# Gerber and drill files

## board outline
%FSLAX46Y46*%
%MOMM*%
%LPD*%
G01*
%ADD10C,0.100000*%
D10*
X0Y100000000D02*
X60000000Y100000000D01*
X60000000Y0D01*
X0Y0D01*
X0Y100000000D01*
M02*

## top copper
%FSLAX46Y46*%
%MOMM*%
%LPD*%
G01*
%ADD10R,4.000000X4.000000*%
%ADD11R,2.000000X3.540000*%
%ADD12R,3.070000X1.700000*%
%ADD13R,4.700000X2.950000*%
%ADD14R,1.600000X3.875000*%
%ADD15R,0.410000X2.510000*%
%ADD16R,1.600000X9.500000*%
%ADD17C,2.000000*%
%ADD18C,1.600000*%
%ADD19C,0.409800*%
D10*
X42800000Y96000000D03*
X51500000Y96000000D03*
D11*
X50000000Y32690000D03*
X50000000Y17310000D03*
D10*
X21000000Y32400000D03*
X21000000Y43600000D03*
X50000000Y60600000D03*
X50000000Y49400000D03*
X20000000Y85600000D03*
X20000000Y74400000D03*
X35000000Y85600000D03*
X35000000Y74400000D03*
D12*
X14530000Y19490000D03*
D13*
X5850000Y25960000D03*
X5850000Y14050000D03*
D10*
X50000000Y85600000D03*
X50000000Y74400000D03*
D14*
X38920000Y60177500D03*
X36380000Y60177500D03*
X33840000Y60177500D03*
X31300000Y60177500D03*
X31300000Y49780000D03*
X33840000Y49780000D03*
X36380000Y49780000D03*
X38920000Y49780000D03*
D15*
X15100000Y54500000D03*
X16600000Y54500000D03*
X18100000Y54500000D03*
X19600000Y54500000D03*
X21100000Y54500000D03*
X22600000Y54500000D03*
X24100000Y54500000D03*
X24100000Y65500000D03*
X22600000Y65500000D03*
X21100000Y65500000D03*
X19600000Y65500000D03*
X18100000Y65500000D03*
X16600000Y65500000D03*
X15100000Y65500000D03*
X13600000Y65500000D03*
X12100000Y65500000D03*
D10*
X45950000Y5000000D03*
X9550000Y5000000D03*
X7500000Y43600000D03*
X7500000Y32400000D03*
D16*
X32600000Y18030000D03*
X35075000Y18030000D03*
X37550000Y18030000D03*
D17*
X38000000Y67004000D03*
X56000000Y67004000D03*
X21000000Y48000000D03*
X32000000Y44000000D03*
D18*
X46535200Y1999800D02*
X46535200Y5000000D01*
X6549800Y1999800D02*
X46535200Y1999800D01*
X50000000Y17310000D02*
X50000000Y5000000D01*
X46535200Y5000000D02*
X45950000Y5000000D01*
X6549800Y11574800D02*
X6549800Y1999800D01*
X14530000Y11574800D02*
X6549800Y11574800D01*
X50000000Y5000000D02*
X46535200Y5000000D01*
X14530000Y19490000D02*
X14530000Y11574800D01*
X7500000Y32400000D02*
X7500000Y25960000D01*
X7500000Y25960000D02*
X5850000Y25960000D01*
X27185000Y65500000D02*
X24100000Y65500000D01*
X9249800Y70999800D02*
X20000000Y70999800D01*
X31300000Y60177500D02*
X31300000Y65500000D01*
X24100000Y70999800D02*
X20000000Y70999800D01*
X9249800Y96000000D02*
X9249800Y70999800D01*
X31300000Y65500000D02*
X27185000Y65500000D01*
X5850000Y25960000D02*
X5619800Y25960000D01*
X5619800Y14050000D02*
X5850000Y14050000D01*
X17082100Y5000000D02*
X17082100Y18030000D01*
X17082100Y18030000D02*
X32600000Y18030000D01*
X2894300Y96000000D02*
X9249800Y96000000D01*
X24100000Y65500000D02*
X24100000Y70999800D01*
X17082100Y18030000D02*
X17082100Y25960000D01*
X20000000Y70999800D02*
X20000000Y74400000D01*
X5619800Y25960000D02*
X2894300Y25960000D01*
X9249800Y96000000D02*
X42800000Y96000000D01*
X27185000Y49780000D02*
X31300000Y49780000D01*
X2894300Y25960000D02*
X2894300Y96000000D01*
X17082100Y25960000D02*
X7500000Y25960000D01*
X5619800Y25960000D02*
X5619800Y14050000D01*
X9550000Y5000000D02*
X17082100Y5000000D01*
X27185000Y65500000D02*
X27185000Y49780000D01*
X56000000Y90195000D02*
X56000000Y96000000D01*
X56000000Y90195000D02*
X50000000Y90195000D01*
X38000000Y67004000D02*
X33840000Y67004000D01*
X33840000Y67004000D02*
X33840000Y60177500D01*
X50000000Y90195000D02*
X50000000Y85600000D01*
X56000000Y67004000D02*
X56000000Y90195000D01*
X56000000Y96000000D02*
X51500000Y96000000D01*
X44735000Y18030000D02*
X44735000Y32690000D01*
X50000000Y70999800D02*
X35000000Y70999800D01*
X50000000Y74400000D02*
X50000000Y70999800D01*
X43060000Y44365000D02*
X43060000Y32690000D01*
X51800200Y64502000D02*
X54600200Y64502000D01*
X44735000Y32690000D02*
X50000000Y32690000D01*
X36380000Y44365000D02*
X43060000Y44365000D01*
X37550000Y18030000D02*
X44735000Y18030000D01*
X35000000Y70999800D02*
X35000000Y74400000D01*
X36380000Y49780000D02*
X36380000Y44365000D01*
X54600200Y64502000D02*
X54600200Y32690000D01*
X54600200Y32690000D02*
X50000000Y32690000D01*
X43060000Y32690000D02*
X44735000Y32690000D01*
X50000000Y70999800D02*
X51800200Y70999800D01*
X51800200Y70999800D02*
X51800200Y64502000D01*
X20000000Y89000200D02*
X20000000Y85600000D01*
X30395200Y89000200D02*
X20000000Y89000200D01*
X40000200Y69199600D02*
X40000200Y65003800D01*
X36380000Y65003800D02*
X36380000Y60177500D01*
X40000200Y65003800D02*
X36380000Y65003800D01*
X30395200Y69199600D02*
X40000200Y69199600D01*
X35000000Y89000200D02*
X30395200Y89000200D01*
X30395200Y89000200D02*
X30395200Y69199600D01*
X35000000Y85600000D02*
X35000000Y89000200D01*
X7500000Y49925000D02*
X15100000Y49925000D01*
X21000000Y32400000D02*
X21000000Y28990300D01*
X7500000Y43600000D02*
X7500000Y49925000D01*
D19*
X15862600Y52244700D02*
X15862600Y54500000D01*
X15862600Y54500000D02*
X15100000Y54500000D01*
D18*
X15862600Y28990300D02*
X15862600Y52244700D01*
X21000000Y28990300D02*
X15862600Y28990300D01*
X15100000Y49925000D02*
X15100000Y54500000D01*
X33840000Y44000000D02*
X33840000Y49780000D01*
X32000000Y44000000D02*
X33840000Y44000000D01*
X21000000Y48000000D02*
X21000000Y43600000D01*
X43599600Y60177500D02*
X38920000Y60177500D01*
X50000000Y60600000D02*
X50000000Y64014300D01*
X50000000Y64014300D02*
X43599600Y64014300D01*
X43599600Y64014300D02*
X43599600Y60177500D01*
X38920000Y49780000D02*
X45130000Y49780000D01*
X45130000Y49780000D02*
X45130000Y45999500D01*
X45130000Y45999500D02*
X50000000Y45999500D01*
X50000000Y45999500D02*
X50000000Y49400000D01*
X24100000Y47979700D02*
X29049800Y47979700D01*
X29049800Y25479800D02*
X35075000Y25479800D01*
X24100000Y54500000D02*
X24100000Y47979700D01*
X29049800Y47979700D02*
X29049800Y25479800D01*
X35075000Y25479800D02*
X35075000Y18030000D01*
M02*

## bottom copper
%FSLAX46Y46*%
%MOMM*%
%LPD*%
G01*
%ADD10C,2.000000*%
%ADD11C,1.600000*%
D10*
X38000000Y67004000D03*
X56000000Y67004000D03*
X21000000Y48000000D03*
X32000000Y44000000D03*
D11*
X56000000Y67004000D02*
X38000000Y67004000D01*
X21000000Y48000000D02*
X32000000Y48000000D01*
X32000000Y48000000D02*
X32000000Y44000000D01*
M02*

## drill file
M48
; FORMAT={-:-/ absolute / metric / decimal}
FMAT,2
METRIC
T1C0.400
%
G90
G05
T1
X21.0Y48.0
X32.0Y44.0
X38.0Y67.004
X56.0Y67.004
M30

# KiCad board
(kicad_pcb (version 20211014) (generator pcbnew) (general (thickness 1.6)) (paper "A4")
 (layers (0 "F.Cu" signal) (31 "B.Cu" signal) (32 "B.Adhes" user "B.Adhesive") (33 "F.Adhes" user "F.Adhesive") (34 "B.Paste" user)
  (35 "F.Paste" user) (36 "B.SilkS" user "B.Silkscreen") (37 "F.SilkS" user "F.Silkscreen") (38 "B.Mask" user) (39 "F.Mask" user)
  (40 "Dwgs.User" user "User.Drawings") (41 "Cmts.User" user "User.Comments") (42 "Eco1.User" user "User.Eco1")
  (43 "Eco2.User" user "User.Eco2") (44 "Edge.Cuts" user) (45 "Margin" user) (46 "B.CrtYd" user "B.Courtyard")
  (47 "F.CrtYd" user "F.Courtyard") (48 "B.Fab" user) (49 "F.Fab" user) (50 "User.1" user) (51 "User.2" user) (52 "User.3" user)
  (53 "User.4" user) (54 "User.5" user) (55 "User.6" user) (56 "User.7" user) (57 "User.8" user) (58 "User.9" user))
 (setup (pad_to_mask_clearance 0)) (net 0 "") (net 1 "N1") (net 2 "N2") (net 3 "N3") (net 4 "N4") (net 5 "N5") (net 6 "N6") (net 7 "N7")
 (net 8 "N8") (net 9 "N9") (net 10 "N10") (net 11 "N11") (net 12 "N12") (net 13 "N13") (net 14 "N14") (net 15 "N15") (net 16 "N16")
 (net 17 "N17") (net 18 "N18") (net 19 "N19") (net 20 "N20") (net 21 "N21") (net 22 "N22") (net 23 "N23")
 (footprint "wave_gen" (layer "F.Cu") (at 47.15 -96 -90)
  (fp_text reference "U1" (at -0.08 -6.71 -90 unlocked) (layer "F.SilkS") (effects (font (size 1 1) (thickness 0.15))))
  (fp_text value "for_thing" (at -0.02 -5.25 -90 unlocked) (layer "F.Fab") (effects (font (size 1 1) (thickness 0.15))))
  (pad "1" smd rect (at 0 4.35 270) (size 4 4) (layers "F.Cu" "F.Paste" "F.Mask") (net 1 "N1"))
  (pad "2" smd rect (at 0 -4.35 90) (size 4 4) (layers "F.Cu" "F.Paste" "F.Mask") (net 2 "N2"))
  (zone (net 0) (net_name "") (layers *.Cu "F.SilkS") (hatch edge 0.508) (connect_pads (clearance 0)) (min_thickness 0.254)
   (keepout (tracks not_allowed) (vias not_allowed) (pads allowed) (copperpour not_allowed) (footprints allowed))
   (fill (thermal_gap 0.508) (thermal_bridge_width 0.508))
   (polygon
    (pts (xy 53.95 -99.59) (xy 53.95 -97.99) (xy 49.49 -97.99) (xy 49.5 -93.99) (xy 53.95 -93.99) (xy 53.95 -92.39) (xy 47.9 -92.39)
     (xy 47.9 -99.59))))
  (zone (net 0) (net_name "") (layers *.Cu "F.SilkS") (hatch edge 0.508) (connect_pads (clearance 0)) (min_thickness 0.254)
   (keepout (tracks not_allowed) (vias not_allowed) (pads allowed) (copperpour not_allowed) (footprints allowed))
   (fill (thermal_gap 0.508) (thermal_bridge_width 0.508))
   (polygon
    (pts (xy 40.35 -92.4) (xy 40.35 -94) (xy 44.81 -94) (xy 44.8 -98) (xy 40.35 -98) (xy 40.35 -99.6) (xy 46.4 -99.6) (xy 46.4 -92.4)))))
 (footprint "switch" (layer "F.Cu") (at 50 -25 -90)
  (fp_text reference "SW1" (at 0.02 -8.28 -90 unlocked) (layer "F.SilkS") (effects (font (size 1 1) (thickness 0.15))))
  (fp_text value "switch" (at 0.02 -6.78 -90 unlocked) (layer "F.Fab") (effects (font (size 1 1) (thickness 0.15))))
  (pad "1" smd rect (at -7.69 0 270) (size 3.54 2) (layers "F.Cu" "F.Paste" "F.Mask") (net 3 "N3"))
  (pad "2" smd rect (at 7.69 0 270) (size 3.54 2) (layers "F.Cu" "F.Paste" "F.Mask") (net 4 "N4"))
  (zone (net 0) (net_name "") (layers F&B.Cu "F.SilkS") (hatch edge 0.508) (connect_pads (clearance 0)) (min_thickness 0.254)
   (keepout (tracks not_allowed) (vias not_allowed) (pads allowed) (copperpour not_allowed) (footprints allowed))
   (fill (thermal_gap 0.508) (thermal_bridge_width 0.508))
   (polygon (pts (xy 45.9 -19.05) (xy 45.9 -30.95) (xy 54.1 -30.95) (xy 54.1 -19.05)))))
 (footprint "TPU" (layer "F.Cu") (at 21 -38 90)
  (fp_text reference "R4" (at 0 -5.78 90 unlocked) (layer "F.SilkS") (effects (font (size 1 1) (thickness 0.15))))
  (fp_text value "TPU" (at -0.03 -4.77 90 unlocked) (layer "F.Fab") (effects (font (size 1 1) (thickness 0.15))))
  (pad "1" smd rect (at -5.6 0 90) (size 4 4) (layers "F.Cu" "F.Paste" "F.Mask") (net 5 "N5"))
  (pad "2" smd rect (at 5.6 0 90) (size 4 4) (layers "F.Cu" "F.Paste" "F.Mask") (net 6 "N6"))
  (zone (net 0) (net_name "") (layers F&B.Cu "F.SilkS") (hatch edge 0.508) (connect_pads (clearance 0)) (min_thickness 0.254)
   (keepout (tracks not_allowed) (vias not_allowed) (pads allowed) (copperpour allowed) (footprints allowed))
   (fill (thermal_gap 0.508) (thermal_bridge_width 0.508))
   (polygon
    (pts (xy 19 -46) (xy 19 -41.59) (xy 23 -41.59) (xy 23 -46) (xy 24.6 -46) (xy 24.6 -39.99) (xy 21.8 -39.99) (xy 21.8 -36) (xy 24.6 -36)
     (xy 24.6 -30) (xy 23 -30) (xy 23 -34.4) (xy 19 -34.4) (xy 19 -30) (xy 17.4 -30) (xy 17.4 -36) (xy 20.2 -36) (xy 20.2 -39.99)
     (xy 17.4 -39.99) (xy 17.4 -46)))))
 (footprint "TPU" (layer "F.Cu") (at 50 -55 -90)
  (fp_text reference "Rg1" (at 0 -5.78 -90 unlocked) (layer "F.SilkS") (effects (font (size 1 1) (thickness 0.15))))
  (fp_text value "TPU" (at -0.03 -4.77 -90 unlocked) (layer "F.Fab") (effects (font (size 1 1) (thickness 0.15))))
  (pad "1" smd rect (at -5.6 0 270) (size 4 4) (layers "F.Cu" "F.Paste" "F.Mask") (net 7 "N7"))
  (pad "2" smd rect (at 5.6 0 270) (size 4 4) (layers "F.Cu" "F.Paste" "F.Mask") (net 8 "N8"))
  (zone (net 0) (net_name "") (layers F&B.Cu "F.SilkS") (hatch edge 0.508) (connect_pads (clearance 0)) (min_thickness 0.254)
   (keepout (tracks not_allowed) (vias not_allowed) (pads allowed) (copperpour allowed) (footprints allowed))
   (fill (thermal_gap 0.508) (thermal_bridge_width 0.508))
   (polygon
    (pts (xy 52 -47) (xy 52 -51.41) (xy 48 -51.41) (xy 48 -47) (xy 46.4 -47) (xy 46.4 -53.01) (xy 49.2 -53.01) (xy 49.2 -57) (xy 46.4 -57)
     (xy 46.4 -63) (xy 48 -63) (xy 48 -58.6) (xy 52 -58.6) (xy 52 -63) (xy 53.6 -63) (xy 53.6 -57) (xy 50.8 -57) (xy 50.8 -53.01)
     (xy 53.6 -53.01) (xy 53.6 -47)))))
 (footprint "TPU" (layer "F.Cu") (at 20 -80 -90)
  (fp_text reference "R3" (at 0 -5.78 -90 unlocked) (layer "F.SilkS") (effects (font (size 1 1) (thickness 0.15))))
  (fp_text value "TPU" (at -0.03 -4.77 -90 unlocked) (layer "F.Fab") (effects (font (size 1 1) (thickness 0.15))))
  (pad "1" smd rect (at -5.6 0 270) (size 4 4) (layers "F.Cu" "F.Paste" "F.Mask") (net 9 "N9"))
  (pad "2" smd rect (at 5.6 0 270) (size 4 4) (layers "F.Cu" "F.Paste" "F.Mask") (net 1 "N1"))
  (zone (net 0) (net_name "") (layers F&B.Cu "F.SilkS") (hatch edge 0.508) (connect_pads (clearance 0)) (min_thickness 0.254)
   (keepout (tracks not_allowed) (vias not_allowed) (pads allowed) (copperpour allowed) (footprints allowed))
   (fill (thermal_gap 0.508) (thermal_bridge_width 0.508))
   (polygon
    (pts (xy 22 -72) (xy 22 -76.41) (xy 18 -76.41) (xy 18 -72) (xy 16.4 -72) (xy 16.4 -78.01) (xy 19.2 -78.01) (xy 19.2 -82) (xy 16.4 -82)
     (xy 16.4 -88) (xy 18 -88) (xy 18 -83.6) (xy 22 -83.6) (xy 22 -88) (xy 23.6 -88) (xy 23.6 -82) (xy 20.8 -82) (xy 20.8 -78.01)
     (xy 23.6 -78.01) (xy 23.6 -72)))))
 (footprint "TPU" (layer "F.Cu") (at 35 -80 -90)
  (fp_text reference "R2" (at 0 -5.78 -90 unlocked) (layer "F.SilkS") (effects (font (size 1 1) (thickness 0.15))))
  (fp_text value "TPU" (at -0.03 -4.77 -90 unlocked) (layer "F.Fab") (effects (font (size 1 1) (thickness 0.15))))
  (pad "1" smd rect (at -5.6 0 270) (size 4 4) (layers "F.Cu" "F.Paste" "F.Mask") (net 9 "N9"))
  (pad "2" smd rect (at 5.6 0 270) (size 4 4) (layers "F.Cu" "F.Paste" "F.Mask") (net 3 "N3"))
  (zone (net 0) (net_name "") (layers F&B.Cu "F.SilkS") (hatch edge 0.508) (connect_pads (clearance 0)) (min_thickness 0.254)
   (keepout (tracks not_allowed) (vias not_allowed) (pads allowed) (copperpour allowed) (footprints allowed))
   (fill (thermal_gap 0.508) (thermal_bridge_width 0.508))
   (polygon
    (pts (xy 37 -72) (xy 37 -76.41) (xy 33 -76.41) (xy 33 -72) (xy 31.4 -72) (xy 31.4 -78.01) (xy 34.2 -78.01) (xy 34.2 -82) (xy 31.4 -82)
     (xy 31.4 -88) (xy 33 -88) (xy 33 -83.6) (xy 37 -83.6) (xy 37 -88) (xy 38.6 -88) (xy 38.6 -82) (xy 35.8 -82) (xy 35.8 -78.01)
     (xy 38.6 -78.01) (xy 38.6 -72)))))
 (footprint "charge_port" (layer "F.Cu") (at 6 -20 180)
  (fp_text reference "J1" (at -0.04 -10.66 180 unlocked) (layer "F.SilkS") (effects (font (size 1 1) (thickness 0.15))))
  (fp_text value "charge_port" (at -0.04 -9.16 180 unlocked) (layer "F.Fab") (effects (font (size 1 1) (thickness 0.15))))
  (pad "1" smd rect (at -8.53 -0.51) (size 3.07 1.7) (layers "F.Cu" "F.Paste" "F.Mask") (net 4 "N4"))
  (pad "2" smd rect (at 0.15 5.96) (size 4.7 2.95) (layers "F.Cu" "F.Paste" "F.Mask") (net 1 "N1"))
  (pad "3" smd rect (at 0.15 -5.95) (size 4.7 2.95) (layers "F.Cu" "F.Paste" "F.Mask") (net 1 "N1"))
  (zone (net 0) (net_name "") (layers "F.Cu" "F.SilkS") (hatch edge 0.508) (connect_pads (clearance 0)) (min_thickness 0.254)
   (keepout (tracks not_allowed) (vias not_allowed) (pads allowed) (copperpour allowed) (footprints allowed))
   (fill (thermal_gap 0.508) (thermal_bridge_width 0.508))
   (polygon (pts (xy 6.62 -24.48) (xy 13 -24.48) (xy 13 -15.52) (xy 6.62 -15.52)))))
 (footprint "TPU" (layer "F.Cu") (at 50 -80 -90)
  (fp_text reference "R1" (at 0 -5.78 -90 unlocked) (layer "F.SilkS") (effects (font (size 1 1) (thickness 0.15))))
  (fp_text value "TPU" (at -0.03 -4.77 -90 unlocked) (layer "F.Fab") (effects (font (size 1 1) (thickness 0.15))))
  (pad "1" smd rect (at -5.6 0 270) (size 4 4) (layers "F.Cu" "F.Paste" "F.Mask") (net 2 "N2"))
  (pad "2" smd rect (at 5.6 0 270) (size 4 4) (layers "F.Cu" "F.Paste" "F.Mask") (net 3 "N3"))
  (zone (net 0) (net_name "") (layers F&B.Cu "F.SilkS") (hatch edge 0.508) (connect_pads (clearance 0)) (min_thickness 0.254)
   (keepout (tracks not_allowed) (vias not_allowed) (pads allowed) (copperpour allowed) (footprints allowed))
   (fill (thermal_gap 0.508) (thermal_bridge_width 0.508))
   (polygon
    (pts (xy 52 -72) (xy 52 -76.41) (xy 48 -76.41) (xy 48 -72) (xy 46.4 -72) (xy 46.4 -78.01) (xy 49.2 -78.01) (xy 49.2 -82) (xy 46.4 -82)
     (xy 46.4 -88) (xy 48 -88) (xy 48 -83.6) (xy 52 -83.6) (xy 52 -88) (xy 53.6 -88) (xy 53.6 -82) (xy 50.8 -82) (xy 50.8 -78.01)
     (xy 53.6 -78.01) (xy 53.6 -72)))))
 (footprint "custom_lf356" (layer "F.Cu") (at 35 -55 -90)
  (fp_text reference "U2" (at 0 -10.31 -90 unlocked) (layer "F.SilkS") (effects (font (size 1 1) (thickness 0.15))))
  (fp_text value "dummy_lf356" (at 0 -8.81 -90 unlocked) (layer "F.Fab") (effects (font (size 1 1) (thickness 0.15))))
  (pad "1" smd rect (at -5.1775 -3.92 270) (size 3.875 1.6) (layers "F.Cu" "F.Paste" "F.Mask") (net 7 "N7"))
  (pad "2" smd rect (at -5.1775 -1.38 270) (size 3.875 1.6) (layers "F.Cu" "F.Paste" "F.Mask") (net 9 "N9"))
  (pad "3" smd rect (at -5.1775 1.16 270) (size 3.875 1.6) (layers "F.Cu" "F.Paste" "F.Mask") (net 2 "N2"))
  (pad "4" smd rect (at -5.1775 3.7 270) (size 3.875 1.6) (layers "F.Cu" "F.Paste" "F.Mask") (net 1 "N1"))
  (pad "5" smd rect (at 5.22 3.7 270) (size 3.875 1.6) (layers "F.Cu" "F.Paste" "F.Mask") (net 1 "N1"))
  (pad "6" smd rect (at 5.22 1.16 270) (size 3.875 1.6) (layers "F.Cu" "F.Paste" "F.Mask") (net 6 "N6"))
  (pad "7" smd rect (at 5.22 -1.38 270) (size 3.875 1.6) (layers "F.Cu" "F.Paste" "F.Mask") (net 3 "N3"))
  (pad "8" smd rect (at 5.22 -3.92 270) (size 3.875 1.6) (layers "F.Cu" "F.Paste" "F.Mask") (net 8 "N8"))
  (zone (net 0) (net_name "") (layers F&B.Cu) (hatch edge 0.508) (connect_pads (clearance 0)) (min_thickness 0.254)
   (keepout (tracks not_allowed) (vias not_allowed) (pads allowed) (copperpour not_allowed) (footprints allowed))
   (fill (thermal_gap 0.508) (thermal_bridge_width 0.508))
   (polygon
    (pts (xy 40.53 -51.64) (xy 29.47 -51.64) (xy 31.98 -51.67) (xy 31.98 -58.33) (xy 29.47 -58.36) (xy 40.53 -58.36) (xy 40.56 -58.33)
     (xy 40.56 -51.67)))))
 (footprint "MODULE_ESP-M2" (layer "F.Cu") (at 15 -60 90) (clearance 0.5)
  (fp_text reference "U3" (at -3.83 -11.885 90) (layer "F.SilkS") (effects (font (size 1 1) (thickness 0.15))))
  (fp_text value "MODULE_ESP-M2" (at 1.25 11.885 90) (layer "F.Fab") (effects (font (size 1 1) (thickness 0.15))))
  (pad "1" smd rect (at -5.5 0.1 90) (size 2.51 0.41) (layers "F.Cu" "F.Paste" "F.Mask") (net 5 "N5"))
  (pad "2" smd rect (at -5.5 1.6 90) (size 2.51 0.41) (layers "F.Cu" "F.Paste" "F.Mask") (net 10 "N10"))
  (pad "3" smd rect (at -5.5 3.1 90) (size 2.51 0.41) (layers "F.Cu" "F.Paste" "F.Mask") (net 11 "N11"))
  (pad "4" smd rect (at -5.5 4.6 90) (size 2.51 0.41) (layers "F.Cu" "F.Paste" "F.Mask") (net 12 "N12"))
  (pad "5" smd rect (at -5.5 6.1 90) (size 2.51 0.41) (layers "F.Cu" "F.Paste" "F.Mask") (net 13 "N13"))
  (pad "6" smd rect (at -5.5 7.6 90) (size 2.51 0.41) (layers "F.Cu" "F.Paste" "F.Mask") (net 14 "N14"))
  (pad "7" smd rect (at -5.5 9.1 90) (size 2.51 0.41) (layers "F.Cu" "F.Paste" "F.Mask") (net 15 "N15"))
  (pad "8" smd rect (at 5.5 9.1 90) (size 2.51 0.41) (layers "F.Cu" "F.Paste" "F.Mask") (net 1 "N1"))
  (pad "9" smd rect (at 5.5 7.6 90) (size 2.51 0.41) (layers "F.Cu" "F.Paste" "F.Mask") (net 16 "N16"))
  (pad "10" smd rect (at 5.5 6.1 90) (size 2.51 0.41) (layers "F.Cu" "F.Paste" "F.Mask") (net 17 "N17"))
  (pad "11" smd rect (at 5.5 4.6 90) (size 2.51 0.41) (layers "F.Cu" "F.Paste" "F.Mask") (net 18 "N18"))
  (pad "12" smd rect (at 5.5 3.1 90) (size 2.51 0.41) (layers "F.Cu" "F.Paste" "F.Mask") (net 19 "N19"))
  (pad "13" smd rect (at 5.5 1.6 90) (size 2.51 0.41) (layers "F.Cu" "F.Paste" "F.Mask") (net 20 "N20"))
  (pad "14" smd rect (at 5.5 0.1 90) (size 2.51 0.41) (layers "F.Cu" "F.Paste" "F.Mask") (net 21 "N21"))
  (pad "15" smd rect (at 5.5 -1.4 90) (size 2.51 0.41) (layers "F.Cu" "F.Paste" "F.Mask") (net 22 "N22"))
  (pad "16" smd rect (at 5.5 -2.9 90) (size 2.51 0.41) (layers "F.Cu" "F.Paste" "F.Mask") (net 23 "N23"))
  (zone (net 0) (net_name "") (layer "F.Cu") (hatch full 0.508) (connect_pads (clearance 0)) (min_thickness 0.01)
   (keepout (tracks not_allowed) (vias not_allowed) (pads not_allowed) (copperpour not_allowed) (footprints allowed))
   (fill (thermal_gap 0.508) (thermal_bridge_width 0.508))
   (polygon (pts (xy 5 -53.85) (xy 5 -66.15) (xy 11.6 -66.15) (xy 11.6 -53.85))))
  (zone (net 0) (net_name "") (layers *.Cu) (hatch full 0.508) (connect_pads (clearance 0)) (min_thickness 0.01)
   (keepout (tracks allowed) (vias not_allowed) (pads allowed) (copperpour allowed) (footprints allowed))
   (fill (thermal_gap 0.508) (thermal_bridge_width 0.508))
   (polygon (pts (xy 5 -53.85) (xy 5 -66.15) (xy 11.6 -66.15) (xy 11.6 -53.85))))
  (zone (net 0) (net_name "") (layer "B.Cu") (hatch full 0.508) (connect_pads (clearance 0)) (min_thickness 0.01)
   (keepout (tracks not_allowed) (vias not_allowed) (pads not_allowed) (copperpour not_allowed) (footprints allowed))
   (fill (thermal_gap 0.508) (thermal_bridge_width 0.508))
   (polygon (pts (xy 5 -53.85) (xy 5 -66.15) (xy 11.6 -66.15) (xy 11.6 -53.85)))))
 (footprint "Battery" (layer "F.Cu") (at 27.75 -5 90)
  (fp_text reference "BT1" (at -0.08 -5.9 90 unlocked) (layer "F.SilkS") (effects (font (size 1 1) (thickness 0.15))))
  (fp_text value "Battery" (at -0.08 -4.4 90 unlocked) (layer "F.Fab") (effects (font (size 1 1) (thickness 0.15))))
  (pad "1" smd rect (at 0 18.2 90) (size 4 4) (layers "F.Cu" "F.Paste" "F.Mask") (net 4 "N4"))
  (pad "2" smd rect (at 0 -18.2 90) (size 4 4) (layers "F.Cu" "F.Paste" "F.Mask") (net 1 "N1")))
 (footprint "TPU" (layer "F.Cu") (at 7.5 -38 -90)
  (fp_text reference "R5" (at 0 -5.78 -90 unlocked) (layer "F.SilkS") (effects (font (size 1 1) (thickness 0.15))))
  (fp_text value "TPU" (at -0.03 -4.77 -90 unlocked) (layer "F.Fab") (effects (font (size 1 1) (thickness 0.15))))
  (pad "1" smd rect (at -5.6 0 270) (size 4 4) (layers "F.Cu" "F.Paste" "F.Mask") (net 5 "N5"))
  (pad "2" smd rect (at 5.6 0 270) (size 4 4) (layers "F.Cu" "F.Paste" "F.Mask") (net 1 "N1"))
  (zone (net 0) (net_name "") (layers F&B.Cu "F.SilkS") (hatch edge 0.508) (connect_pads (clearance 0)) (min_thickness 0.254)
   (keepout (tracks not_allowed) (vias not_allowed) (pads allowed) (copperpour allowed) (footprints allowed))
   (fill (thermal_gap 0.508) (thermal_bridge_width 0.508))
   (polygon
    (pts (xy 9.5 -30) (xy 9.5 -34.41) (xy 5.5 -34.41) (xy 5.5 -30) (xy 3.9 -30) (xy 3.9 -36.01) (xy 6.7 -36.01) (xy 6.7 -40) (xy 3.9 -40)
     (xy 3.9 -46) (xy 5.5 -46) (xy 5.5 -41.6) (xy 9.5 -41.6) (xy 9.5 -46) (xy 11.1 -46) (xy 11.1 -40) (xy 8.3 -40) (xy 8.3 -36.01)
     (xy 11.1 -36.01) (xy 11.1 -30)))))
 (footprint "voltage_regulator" (layer "F.Cu") (at 35 -28 -90)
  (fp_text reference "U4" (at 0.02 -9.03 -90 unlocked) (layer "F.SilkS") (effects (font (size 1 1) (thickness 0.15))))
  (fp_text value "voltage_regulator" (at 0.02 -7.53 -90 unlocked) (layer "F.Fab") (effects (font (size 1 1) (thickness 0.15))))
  (pad "1" smd rect (at 9.97 2.4 270) (size 9.5 1.6) (layers "F.Cu" "F.Paste" "F.Mask") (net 1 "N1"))
  (pad "2" smd rect (at 9.97 -0.075 270) (size 9.5 1.6) (layers "F.Cu" "F.Paste" "F.Mask") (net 15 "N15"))
  (pad "3" smd rect (at 9.97 -2.55 270) (size 9.5 1.6) (layers "F.Cu" "F.Paste" "F.Mask") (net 3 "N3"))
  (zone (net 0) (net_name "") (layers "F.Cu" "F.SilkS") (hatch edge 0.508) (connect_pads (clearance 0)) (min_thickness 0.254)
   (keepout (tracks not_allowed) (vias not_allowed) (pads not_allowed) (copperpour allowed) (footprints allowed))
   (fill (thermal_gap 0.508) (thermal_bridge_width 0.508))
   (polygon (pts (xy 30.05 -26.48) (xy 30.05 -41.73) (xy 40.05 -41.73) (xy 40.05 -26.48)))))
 (gr_rect (start 0 0) (end 60 -100) (layer "Edge.Cuts") (width 0.1) (fill none))
 (segment (start 46.5352 -1.9998) (end 46.5352 -5) (width 1.6) (layer "F.Cu") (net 4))
 (segment (start 6.5498 -1.9998) (end 46.5352 -1.9998) (width 1.6) (layer "F.Cu") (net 4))
 (segment (start 50 -17.31) (end 50 -5) (width 1.6) (layer "F.Cu") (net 4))
 (segment (start 46.5352 -5) (end 45.95 -5) (width 1.6) (layer "F.Cu") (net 4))
 (segment (start 6.5498 -11.5748) (end 6.5498 -1.9998) (width 1.6) (layer "F.Cu") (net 4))
 (segment (start 14.53 -11.5748) (end 6.5498 -11.5748) (width 1.6) (layer "F.Cu") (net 4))
 (segment (start 50 -5) (end 46.5352 -5) (width 1.6) (layer "F.Cu") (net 4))
 (segment (start 14.53 -19.49) (end 14.53 -11.5748) (width 1.6) (layer "F.Cu") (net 4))
 (segment (start 7.5 -32.4) (end 7.5 -25.96) (width 1.6) (layer "F.Cu") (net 1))
 (segment (start 7.5 -25.96) (end 5.85 -25.96) (width 1.6) (layer "F.Cu") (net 1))
 (segment (start 27.185 -65.5) (end 24.1 -65.5) (width 1.6) (layer "F.Cu") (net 1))
 (segment (start 9.2498 -70.9998) (end 20 -70.9998) (width 1.6) (layer "F.Cu") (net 1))
 (segment (start 31.3 -60.1775) (end 31.3 -65.5) (width 1.6) (layer "F.Cu") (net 1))
 (segment (start 24.1 -70.9998) (end 20 -70.9998) (width 1.6) (layer "F.Cu") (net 1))
 (segment (start 9.2498 -96) (end 9.2498 -70.9998) (width 1.6) (layer "F.Cu") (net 1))
 (segment (start 31.3 -65.5) (end 27.185 -65.5) (width 1.6) (layer "F.Cu") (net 1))
 (segment (start 5.85 -25.96) (end 5.6198 -25.96) (width 1.6) (layer "F.Cu") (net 1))
 (segment (start 5.6198 -14.05) (end 5.85 -14.05) (width 1.6) (layer "F.Cu") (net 1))
 (segment (start 17.0821 -5) (end 17.0821 -18.03) (width 1.6) (layer "F.Cu") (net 1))
 (segment (start 17.0821 -18.03) (end 32.6 -18.03) (width 1.6) (layer "F.Cu") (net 1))
 (segment (start 2.8943 -96) (end 9.2498 -96) (width 1.6) (layer "F.Cu") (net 1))
 (segment (start 24.1 -65.5) (end 24.1 -70.9998) (width 1.6) (layer "F.Cu") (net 1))
 (segment (start 17.0821 -18.03) (end 17.0821 -25.96) (width 1.6) (layer "F.Cu") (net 1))
 (segment (start 20 -70.9998) (end 20 -74.4) (width 1.6) (layer "F.Cu") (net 1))
 (segment (start 5.6198 -25.96) (end 2.8943 -25.96) (width 1.6) (layer "F.Cu") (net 1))
 (segment (start 9.2498 -96) (end 42.8 -96) (width 1.6) (layer "F.Cu") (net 1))
 (segment (start 27.185 -49.78) (end 31.3 -49.78) (width 1.6) (layer "F.Cu") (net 1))
 (segment (start 2.8943 -25.96) (end 2.8943 -96) (width 1.6) (layer "F.Cu") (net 1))
 (segment (start 17.0821 -25.96) (end 7.5 -25.96) (width 1.6) (layer "F.Cu") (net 1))
 (segment (start 5.6198 -25.96) (end 5.6198 -14.05) (width 1.6) (layer "F.Cu") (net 1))
 (segment (start 9.55 -5) (end 17.0821 -5) (width 1.6) (layer "F.Cu") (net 1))
 (segment (start 27.185 -65.5) (end 27.185 -49.78) (width 1.6) (layer "F.Cu") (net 1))
 (segment (start 56 -90.195) (end 56 -96) (width 1.6) (layer "F.Cu") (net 2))
 (segment (start 56 -90.195) (end 50 -90.195) (width 1.6) (layer "F.Cu") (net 2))
 (segment (start 38 -67.004) (end 33.84 -67.004) (width 1.6) (layer "F.Cu") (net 2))
 (segment (start 33.84 -67.004) (end 33.84 -60.1775) (width 1.6) (layer "F.Cu") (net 2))
 (segment (start 50 -90.195) (end 50 -85.6) (width 1.6) (layer "F.Cu") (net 2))
 (segment (start 56 -67.004) (end 56 -90.195) (width 1.6) (layer "F.Cu") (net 2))
 (segment (start 56 -96) (end 51.5 -96) (width 1.6) (layer "F.Cu") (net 2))
 (via (at 38 -67.004) (size 2) (drill 0.4) (layers "F.Cu" "B.Cu") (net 2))
 (via (at 56 -67.004) (size 2) (drill 0.4) (layers "F.Cu" "B.Cu") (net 2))
 (segment (start 56 -67.004) (end 38 -67.004) (width 1.6) (layer "B.Cu") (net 2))
 (segment (start 44.735 -18.03) (end 44.735 -32.69) (width 1.6) (layer "F.Cu") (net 3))
 (segment (start 50 -70.9998) (end 35 -70.9998) (width 1.6) (layer "F.Cu") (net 3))
 (segment (start 50 -74.4) (end 50 -70.9998) (width 1.6) (layer "F.Cu") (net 3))
 (segment (start 43.06 -44.365) (end 43.06 -32.69) (width 1.6) (layer "F.Cu") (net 3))
 (segment (start 51.8002 -64.502) (end 54.6002 -64.502) (width 1.6) (layer "F.Cu") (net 3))
 (segment (start 44.735 -32.69) (end 50 -32.69) (width 1.6) (layer "F.Cu") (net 3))
 (segment (start 36.38 -44.365) (end 43.06 -44.365) (width 1.6) (layer "F.Cu") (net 3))
 (segment (start 37.55 -18.03) (end 44.735 -18.03) (width 1.6) (layer "F.Cu") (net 3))
 (segment (start 35 -70.9998) (end 35 -74.4) (width 1.6) (layer "F.Cu") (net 3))
 (segment (start 36.38 -49.78) (end 36.38 -44.365) (width 1.6) (layer "F.Cu") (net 3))
 (segment (start 54.6002 -64.502) (end 54.6002 -32.69) (width 1.6) (layer "F.Cu") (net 3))
 (segment (start 54.6002 -32.69) (end 50 -32.69) (width 1.6) (layer "F.Cu") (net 3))
 (segment (start 43.06 -32.69) (end 44.735 -32.69) (width 1.6) (layer "F.Cu") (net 3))
 (segment (start 50 -70.9998) (end 51.8002 -70.9998) (width 1.6) (layer "F.Cu") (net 3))
 (segment (start 51.8002 -70.9998) (end 51.8002 -64.502) (width 1.6) (layer "F.Cu") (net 3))
 (segment (start 20 -89.0002) (end 20 -85.6) (width 1.6) (layer "F.Cu") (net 9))
 (segment (start 30.3952 -89.0002) (end 20 -89.0002) (width 1.6) (layer "F.Cu") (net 9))
 (segment (start 40.0002 -69.1996) (end 40.0002 -65.0038) (width 1.6) (layer "F.Cu") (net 9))
 (segment (start 36.38 -65.0038) (end 36.38 -60.1775) (width 1.6) (layer "F.Cu") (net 9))
 (segment (start 40.0002 -65.0038) (end 36.38 -65.0038) (width 1.6) (layer "F.Cu") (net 9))
 (segment (start 30.3952 -69.1996) (end 40.0002 -69.1996) (width 1.6) (layer "F.Cu") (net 9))
 (segment (start 35 -89.0002) (end 30.3952 -89.0002) (width 1.6) (layer "F.Cu") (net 9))
 (segment (start 30.3952 -89.0002) (end 30.3952 -69.1996) (width 1.6) (layer "F.Cu") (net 9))
 (segment (start 35 -85.6) (end 35 -89.0002) (width 1.6) (layer "F.Cu") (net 9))
 (segment (start 7.5 -49.925) (end 15.1 -49.925) (width 1.6) (layer "F.Cu") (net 5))
 (segment (start 21 -32.4) (end 21 -28.9903) (width 1.6) (layer "F.Cu") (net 5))
 (segment (start 7.5 -43.6) (end 7.5 -49.925) (width 1.6) (layer "F.Cu") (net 5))
 (segment (start 15.8626 -52.2447) (end 15.8626 -54.5) (width 0.4098) (layer "F.Cu") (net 5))
 (segment (start 15.8626 -54.5) (end 15.1 -54.5) (width 0.4098) (layer "F.Cu") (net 5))
 (segment (start 15.8626 -28.9903) (end 15.8626 -52.2447) (width 1.6) (layer "F.Cu") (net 5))
 (segment (start 21 -28.9903) (end 15.8626 -28.9903) (width 1.6) (layer "F.Cu") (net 5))
 (segment (start 15.1 -49.925) (end 15.1 -54.5) (width 1.6) (layer "F.Cu") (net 5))
 (segment (start 33.84 -44) (end 33.84 -49.78) (width 1.6) (layer "F.Cu") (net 6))
 (segment (start 32 -44) (end 33.84 -44) (width 1.6) (layer "F.Cu") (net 6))
 (segment (start 21 -48) (end 21 -43.6) (width 1.6) (layer "F.Cu") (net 6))
 (via (at 21 -48) (size 2) (drill 0.4) (layers "F.Cu" "B.Cu") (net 6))
 (via (at 32 -44) (size 2) (drill 0.4) (layers "F.Cu" "B.Cu") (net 6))
 (segment (start 21 -48) (end 32 -48) (width 1.6) (layer "B.Cu") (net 6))
 (segment (start 32 -48) (end 32 -44) (width 1.6) (layer "B.Cu") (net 6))
 (segment (start 43.5996 -60.1775) (end 38.92 -60.1775) (width 1.6) (layer "F.Cu") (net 7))
 (segment (start 50 -60.6) (end 50 -64.0143) (width 1.6) (layer "F.Cu") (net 7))
 (segment (start 50 -64.0143) (end 43.5996 -64.0143) (width 1.6) (layer "F.Cu") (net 7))
 (segment (start 43.5996 -64.0143) (end 43.5996 -60.1775) (width 1.6) (layer "F.Cu") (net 7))
 (segment (start 38.92 -49.78) (end 45.13 -49.78) (width 1.6) (layer "F.Cu") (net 8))
 (segment (start 45.13 -49.78) (end 45.13 -45.9995) (width 1.6) (layer "F.Cu") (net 8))
 (segment (start 45.13 -45.9995) (end 50 -45.9995) (width 1.6) (layer "F.Cu") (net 8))
 (segment (start 50 -45.9995) (end 50 -49.4) (width 1.6) (layer "F.Cu") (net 8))
 (segment (start 24.1 -47.9797) (end 29.0498 -47.9797) (width 1.6) (layer "F.Cu") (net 15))
 (segment (start 29.0498 -25.4798) (end 35.075 -25.4798) (width 1.6) (layer "F.Cu") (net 15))
 (segment (start 24.1 -54.5) (end 24.1 -47.9797) (width 1.6) (layer "F.Cu") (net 15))
 (segment (start 29.0498 -47.9797) (end 29.0498 -25.4798) (width 1.6) (layer "F.Cu") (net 15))
 (segment (start 35.075 -25.4798) (end 35.075 -18.03) (width 1.6) (layer "F.Cu") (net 15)))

